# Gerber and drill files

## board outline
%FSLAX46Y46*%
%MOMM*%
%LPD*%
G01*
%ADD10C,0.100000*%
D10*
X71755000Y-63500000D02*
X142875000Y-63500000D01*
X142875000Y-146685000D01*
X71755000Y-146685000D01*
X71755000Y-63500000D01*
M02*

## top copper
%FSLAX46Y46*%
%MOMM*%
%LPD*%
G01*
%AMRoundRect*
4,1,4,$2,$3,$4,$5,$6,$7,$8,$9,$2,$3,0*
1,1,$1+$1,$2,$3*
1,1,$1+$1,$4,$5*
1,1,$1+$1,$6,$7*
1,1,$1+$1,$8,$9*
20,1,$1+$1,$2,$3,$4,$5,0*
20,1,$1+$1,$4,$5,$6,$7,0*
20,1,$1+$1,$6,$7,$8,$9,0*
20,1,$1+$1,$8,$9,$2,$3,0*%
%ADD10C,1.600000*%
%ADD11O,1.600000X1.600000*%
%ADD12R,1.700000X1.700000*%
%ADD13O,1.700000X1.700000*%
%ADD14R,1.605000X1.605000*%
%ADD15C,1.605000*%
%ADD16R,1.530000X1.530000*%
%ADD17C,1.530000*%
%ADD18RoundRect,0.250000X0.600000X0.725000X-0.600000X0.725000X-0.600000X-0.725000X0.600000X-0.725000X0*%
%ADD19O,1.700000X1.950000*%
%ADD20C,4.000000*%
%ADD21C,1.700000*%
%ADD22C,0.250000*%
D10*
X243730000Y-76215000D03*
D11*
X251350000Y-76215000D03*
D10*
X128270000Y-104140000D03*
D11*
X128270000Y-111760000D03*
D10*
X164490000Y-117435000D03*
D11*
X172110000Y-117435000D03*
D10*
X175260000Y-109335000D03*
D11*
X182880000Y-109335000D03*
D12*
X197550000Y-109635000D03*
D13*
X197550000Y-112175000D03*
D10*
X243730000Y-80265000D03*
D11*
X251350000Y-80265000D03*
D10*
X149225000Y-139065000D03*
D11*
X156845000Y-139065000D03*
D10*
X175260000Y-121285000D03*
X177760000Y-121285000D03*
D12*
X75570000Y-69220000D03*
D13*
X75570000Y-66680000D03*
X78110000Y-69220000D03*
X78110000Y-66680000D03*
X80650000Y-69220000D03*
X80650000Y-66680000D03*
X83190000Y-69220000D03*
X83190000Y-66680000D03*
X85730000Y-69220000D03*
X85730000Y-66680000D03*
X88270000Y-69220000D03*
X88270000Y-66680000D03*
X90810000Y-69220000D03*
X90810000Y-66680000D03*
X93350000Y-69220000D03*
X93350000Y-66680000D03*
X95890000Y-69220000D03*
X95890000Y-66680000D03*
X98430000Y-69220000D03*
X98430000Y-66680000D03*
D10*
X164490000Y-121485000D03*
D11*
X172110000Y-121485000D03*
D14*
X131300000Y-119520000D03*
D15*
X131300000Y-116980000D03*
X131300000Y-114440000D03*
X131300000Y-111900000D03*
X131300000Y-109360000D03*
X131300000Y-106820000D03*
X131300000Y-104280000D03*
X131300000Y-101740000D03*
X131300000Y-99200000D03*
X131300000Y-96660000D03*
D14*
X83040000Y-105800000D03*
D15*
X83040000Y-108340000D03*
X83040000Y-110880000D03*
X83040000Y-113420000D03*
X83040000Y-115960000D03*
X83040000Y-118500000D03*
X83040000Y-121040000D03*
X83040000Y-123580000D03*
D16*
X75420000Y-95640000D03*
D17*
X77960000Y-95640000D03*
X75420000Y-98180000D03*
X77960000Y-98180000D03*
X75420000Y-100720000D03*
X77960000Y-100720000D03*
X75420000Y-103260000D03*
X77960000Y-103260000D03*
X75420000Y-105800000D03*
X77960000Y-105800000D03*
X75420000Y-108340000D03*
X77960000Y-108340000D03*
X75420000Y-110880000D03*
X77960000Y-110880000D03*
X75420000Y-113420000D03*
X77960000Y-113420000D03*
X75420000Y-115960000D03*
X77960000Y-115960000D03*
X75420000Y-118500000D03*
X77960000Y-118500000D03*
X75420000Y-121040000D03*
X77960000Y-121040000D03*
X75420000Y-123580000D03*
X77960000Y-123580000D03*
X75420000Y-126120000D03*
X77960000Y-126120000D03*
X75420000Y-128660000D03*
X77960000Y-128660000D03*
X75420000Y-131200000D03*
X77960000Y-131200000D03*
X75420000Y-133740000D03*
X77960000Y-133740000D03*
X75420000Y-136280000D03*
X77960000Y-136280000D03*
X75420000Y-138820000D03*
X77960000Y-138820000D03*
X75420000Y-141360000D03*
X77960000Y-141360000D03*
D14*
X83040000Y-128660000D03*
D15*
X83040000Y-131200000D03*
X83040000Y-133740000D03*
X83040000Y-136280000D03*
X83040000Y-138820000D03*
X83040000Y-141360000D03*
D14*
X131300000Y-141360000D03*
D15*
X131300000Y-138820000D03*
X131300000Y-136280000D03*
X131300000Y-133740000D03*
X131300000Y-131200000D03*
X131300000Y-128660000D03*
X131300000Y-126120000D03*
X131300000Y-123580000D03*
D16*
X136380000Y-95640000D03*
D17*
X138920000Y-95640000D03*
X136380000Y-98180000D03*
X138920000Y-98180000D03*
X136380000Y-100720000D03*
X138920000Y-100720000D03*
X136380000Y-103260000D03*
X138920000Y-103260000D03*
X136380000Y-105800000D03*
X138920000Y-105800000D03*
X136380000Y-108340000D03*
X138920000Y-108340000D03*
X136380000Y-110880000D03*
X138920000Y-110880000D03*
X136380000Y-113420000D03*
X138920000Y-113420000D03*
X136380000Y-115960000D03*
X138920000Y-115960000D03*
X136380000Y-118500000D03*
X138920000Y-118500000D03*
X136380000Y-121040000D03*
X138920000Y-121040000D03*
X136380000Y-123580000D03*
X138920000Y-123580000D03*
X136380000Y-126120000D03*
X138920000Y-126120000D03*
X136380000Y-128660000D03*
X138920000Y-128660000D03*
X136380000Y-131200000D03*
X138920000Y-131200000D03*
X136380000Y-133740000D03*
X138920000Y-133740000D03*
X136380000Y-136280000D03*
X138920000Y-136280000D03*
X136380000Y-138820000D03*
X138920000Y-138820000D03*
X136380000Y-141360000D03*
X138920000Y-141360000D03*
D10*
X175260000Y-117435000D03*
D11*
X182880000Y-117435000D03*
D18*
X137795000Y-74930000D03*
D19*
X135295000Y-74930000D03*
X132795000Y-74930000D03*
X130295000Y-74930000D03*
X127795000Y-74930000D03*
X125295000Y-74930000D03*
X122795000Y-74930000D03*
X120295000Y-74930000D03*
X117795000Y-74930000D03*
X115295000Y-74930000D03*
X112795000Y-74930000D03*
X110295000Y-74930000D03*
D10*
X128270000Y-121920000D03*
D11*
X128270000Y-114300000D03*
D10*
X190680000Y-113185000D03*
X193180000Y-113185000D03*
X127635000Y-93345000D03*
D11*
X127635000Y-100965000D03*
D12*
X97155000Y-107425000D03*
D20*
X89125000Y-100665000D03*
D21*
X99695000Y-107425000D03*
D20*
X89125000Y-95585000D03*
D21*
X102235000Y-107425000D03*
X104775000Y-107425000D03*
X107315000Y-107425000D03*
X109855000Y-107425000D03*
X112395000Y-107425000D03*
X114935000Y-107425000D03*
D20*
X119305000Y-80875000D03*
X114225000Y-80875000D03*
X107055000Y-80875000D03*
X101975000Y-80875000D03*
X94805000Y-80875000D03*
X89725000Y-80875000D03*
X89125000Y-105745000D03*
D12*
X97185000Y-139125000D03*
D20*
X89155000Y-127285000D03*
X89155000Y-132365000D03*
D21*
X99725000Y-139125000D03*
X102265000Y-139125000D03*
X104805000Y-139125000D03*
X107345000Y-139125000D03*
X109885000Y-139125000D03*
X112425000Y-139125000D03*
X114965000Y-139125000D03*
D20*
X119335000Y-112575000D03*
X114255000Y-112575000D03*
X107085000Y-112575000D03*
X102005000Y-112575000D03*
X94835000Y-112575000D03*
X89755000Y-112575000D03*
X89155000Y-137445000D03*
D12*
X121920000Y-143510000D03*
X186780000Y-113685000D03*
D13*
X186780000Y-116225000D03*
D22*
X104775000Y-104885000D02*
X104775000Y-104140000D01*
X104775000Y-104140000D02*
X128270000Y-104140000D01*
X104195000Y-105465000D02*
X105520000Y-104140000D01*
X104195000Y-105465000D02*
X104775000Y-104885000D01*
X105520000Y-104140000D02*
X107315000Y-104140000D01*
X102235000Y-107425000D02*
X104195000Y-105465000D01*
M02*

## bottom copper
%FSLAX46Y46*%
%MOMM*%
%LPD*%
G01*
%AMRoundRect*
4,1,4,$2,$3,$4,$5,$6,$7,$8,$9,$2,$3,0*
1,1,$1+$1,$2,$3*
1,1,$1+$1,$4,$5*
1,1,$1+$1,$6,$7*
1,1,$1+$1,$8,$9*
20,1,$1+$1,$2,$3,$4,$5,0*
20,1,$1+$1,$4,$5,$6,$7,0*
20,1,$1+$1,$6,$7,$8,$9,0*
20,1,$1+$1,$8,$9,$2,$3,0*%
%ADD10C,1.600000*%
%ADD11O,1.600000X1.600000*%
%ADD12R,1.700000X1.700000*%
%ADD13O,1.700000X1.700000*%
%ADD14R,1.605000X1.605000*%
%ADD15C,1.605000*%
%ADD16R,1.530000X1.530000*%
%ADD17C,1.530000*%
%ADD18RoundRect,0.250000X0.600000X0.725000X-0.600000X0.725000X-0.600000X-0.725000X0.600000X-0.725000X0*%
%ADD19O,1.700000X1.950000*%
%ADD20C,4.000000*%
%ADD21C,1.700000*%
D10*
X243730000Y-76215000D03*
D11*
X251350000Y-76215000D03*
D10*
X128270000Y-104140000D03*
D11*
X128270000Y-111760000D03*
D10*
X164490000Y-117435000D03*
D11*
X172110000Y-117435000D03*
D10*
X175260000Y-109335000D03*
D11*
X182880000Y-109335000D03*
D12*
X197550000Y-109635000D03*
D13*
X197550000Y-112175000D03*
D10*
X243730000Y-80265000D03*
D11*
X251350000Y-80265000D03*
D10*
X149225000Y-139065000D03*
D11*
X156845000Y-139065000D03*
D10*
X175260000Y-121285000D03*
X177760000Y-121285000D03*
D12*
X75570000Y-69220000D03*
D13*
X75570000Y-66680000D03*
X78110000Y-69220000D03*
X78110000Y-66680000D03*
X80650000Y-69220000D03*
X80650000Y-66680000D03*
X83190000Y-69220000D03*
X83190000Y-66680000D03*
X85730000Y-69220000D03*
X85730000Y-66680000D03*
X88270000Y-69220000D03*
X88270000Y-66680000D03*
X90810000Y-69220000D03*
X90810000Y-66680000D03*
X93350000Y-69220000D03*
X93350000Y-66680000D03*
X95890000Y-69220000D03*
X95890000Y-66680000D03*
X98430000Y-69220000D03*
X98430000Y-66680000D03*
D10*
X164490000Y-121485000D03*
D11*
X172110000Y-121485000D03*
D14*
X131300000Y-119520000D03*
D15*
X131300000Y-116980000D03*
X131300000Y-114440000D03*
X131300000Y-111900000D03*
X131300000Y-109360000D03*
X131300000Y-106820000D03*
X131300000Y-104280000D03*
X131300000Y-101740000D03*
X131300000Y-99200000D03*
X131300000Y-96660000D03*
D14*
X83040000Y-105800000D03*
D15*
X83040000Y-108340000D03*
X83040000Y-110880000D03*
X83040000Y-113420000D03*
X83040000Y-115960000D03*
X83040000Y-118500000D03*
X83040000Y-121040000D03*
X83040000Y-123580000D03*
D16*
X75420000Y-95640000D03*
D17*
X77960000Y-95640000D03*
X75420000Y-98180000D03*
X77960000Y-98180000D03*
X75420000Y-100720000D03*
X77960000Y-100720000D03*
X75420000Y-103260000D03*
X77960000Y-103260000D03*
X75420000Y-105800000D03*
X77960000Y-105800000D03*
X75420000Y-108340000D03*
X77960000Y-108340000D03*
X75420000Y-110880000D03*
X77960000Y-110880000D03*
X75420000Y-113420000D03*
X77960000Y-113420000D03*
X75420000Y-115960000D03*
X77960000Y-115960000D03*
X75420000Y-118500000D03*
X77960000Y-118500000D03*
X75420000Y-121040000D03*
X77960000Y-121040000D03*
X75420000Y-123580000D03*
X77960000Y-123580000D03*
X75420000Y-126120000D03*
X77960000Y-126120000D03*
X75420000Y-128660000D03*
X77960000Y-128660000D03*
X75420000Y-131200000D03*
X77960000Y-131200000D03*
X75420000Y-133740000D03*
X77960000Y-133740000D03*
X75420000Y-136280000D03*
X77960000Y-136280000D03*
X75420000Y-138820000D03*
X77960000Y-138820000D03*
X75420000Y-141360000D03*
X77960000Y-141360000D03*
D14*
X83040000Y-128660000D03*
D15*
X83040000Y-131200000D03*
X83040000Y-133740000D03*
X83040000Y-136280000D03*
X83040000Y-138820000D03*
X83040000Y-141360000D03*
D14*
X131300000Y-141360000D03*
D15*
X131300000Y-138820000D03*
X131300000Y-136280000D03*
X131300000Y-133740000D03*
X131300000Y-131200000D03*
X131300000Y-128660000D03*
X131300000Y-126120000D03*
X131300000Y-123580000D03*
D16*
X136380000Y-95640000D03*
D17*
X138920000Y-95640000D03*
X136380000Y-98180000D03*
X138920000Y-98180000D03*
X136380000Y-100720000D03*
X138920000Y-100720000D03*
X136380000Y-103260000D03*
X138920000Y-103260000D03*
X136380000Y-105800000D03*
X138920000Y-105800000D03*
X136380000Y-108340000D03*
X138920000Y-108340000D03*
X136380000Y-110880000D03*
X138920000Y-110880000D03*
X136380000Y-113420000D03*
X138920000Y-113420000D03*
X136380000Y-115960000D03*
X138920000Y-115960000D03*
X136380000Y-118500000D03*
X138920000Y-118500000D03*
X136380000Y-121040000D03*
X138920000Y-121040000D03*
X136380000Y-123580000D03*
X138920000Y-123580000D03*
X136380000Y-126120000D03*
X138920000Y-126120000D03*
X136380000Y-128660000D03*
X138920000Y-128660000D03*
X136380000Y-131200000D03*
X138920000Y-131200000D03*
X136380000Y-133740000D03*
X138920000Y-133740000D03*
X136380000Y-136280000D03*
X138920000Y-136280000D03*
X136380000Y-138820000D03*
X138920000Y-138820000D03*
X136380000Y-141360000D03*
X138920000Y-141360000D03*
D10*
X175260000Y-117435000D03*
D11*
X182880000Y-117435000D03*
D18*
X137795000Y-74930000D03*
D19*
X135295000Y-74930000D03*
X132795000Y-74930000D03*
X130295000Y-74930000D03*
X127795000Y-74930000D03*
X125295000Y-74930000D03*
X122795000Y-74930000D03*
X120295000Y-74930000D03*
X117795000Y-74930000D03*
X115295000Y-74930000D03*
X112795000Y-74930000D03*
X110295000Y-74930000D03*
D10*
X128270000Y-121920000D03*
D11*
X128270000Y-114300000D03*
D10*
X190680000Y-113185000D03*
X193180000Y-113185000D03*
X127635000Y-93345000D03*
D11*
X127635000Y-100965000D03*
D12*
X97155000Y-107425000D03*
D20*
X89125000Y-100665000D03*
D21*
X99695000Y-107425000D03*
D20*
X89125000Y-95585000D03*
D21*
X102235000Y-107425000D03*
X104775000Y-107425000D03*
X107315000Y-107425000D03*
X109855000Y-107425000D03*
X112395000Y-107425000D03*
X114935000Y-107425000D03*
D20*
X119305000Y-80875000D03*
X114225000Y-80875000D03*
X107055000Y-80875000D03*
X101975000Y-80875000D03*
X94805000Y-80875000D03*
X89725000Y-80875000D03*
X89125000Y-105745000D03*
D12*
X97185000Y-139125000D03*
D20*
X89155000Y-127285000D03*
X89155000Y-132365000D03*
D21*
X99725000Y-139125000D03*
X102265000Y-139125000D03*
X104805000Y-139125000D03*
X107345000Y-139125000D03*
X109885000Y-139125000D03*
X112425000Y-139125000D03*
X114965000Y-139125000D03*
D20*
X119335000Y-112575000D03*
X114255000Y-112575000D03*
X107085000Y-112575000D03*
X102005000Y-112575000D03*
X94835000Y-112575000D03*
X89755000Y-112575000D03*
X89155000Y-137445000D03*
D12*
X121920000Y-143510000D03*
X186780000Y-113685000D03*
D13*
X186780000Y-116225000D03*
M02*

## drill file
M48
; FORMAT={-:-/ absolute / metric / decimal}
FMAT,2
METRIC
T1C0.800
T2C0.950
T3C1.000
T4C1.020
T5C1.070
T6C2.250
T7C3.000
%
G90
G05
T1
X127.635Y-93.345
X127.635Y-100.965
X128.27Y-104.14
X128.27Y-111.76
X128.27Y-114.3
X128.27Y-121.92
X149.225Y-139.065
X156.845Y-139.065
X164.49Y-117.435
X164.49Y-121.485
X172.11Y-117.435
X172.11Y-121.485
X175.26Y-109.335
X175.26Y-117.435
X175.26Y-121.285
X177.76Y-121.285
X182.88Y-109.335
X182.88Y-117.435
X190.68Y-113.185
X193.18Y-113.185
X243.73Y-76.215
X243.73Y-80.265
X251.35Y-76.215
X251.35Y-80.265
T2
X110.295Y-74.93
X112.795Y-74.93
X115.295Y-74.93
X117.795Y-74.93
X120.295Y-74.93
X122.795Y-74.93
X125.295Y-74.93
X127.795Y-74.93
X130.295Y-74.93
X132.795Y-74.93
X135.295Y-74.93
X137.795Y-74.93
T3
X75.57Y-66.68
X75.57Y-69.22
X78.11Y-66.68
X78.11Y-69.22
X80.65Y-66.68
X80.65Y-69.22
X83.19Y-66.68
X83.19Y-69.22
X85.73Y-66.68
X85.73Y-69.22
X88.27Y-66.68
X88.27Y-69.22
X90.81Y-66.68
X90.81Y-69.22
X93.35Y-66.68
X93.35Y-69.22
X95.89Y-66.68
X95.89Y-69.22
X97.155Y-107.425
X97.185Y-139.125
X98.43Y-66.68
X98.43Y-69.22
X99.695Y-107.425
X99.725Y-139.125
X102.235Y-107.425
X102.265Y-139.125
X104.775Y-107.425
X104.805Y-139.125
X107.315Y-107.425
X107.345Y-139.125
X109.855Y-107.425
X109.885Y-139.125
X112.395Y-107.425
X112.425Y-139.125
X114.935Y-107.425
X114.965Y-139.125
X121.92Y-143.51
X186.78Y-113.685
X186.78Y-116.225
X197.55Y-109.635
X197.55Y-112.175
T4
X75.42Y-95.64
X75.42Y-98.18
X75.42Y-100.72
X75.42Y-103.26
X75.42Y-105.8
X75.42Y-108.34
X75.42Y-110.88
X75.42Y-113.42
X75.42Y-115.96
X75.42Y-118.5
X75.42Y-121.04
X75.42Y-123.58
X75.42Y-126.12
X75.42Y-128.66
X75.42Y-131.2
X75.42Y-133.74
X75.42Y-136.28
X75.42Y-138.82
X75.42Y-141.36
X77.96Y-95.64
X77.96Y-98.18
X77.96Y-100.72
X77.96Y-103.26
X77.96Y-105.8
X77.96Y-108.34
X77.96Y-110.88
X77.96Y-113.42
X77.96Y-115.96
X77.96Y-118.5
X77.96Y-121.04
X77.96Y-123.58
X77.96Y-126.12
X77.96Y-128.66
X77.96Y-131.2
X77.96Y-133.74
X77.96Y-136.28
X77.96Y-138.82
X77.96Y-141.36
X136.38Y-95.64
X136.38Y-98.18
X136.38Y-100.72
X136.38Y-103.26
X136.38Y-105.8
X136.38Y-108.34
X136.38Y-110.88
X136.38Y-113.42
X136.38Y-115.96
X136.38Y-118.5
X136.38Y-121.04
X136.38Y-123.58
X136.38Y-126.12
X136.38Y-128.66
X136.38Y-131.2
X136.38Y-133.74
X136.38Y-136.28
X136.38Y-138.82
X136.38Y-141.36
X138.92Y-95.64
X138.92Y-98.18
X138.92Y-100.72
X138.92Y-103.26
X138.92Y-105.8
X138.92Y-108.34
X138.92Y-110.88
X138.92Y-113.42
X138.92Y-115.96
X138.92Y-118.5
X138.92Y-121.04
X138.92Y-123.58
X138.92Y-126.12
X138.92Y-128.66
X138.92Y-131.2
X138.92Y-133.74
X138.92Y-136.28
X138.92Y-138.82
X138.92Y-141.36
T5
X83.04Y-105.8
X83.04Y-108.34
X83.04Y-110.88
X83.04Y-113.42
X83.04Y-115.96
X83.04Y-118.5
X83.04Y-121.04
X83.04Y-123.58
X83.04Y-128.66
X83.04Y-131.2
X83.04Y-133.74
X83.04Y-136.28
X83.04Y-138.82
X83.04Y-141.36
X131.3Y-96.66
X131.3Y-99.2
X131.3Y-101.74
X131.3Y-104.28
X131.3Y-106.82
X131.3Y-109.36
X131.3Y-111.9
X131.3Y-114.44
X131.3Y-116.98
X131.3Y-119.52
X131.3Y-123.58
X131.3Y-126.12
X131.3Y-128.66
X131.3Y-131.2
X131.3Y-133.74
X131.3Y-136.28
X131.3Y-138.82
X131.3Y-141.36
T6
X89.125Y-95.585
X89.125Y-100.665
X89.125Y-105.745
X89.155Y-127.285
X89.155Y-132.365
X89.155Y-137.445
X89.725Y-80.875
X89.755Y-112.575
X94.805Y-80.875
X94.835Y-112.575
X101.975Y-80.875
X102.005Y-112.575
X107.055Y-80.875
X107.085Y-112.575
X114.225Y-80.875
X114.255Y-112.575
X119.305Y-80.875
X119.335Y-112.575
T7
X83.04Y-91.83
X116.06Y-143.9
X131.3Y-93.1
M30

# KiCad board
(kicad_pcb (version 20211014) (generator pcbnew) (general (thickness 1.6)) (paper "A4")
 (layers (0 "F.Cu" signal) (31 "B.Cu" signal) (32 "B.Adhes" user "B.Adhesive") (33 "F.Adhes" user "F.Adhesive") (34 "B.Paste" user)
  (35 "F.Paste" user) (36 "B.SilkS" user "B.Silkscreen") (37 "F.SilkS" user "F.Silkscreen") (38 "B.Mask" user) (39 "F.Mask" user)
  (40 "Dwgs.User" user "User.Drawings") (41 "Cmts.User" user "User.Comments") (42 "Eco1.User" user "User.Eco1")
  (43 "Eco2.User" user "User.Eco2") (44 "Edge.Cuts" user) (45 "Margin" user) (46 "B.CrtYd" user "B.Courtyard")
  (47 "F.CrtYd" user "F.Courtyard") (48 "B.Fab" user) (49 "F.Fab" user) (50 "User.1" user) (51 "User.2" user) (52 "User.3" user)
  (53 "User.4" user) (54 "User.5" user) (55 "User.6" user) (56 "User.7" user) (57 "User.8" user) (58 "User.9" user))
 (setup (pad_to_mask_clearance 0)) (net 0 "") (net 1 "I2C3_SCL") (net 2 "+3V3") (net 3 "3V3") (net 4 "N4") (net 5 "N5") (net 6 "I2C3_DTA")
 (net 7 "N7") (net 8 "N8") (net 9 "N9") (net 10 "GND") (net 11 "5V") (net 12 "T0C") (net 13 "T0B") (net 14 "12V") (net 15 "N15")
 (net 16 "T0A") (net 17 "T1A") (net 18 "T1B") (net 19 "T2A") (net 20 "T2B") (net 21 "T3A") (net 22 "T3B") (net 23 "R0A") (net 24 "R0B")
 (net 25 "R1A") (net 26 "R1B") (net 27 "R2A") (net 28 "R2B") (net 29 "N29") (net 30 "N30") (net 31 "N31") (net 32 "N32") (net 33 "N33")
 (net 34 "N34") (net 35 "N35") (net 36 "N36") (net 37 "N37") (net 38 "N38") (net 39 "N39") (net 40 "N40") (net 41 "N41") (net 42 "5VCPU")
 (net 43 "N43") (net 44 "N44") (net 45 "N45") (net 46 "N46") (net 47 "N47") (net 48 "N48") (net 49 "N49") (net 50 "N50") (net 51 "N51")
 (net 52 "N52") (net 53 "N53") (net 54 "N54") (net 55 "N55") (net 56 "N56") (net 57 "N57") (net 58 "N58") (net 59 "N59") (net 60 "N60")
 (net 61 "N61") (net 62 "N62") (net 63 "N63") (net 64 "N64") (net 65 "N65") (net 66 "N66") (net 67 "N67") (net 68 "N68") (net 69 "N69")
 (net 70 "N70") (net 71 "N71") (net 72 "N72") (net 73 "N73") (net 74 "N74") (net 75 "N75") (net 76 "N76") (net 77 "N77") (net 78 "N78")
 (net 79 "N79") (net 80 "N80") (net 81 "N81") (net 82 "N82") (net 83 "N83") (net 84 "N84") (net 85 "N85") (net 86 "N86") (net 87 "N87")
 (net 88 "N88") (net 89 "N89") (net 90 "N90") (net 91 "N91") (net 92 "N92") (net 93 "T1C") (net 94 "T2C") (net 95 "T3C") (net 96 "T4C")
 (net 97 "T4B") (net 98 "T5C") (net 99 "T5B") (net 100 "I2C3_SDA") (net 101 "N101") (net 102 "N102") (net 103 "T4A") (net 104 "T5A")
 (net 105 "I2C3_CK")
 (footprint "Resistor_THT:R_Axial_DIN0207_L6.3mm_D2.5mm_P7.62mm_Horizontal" (layer "F.Cu") (at 243.73 76.215)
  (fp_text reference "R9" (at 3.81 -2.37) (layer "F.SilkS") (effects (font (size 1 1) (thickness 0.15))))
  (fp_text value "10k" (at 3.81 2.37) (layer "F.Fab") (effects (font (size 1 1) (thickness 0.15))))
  (pad "1" thru_hole circle (at 0 0) (size 1.6 1.6) (drill 0.8) (layers *.Cu *.Mask) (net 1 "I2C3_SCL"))
  (pad "2" thru_hole oval (at 7.62 0) (size 1.6 1.6) (drill 0.8) (layers *.Cu *.Mask) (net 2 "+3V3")))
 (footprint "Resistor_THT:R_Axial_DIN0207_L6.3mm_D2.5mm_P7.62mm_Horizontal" (layer "F.Cu") (at 128.27 104.14 -90)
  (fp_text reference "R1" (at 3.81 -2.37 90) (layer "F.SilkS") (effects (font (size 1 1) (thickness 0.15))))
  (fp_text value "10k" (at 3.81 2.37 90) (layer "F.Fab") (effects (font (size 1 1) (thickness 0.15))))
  (pad "1" thru_hole circle (at 0 0 270) (size 1.6 1.6) (drill 0.8) (layers *.Cu *.Mask) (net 1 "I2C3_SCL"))
  (pad "2" thru_hole oval (at 7.62 0 270) (size 1.6 1.6) (drill 0.8) (layers *.Cu *.Mask) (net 2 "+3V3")))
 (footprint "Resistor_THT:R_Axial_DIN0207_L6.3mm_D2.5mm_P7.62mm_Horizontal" (layer "F.Cu") (at 164.49 117.435)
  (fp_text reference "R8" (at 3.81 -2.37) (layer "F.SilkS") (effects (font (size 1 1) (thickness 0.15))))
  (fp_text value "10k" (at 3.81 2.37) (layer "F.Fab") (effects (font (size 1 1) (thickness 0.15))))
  (pad "1" thru_hole circle (at 0 0) (size 1.6 1.6) (drill 0.8) (layers *.Cu *.Mask) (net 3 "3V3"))
  (pad "2" thru_hole oval (at 7.62 0) (size 1.6 1.6) (drill 0.8) (layers *.Cu *.Mask) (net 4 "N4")))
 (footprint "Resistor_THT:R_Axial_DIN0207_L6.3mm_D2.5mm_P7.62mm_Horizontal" (layer "F.Cu") (at 175.26 109.335)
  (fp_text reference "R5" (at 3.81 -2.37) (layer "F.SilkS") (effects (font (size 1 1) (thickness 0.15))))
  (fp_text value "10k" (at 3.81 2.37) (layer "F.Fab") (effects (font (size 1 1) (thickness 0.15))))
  (pad "1" thru_hole circle (at 0 0) (size 1.6 1.6) (drill 0.8) (layers *.Cu *.Mask) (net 3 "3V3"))
  (pad "2" thru_hole oval (at 7.62 0) (size 1.6 1.6) (drill 0.8) (layers *.Cu *.Mask) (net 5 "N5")))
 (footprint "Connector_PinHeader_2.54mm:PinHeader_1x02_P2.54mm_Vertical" (layer "F.Cu") (at 197.55 109.635)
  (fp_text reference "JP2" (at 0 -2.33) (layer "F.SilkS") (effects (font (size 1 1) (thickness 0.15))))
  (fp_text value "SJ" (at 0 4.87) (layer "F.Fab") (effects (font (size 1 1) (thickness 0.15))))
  (pad "1" thru_hole rect (at 0 0) (size 1.7 1.7) (drill 1) (layers *.Cu *.Mask) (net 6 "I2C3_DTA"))
  (pad "2" thru_hole oval (at 0 2.54) (size 1.7 1.7) (drill 1) (layers *.Cu *.Mask) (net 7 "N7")))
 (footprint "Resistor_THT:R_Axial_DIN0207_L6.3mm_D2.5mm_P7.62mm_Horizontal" (layer "F.Cu") (at 243.73 80.265)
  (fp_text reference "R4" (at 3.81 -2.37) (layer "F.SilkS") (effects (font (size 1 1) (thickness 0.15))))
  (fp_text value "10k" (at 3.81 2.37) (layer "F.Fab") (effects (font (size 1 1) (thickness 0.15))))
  (pad "1" thru_hole circle (at 0 0) (size 1.6 1.6) (drill 0.8) (layers *.Cu *.Mask) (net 3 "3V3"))
  (pad "2" thru_hole oval (at 7.62 0) (size 1.6 1.6) (drill 0.8) (layers *.Cu *.Mask) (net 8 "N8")))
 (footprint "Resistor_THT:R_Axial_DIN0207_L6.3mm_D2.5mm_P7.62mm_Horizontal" (layer "F.Cu") (at 149.225 139.065)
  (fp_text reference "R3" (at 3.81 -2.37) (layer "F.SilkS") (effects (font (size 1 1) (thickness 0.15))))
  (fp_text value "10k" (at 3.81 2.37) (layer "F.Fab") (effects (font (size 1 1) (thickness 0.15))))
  (pad "1" thru_hole circle (at 0 0) (size 1.6 1.6) (drill 0.8) (layers *.Cu *.Mask) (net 3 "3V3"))
  (pad "2" thru_hole oval (at 7.62 0) (size 1.6 1.6) (drill 0.8) (layers *.Cu *.Mask) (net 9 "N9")))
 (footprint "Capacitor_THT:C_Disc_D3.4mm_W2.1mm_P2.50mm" (layer "F.Cu") (at 175.26 121.285)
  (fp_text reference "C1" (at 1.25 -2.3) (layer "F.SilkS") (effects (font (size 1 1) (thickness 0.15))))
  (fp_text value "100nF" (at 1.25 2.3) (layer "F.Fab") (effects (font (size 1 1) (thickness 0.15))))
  (pad "1" thru_hole circle (at 0 0) (size 1.6 1.6) (drill 0.8) (layers *.Cu *.Mask) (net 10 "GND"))
  (pad "2" thru_hole circle (at 2.5 0) (size 1.6 1.6) (drill 0.8) (layers *.Cu *.Mask) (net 3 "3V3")))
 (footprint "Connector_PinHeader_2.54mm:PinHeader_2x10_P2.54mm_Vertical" (layer "F.Cu") (at 75.57 69.22 90)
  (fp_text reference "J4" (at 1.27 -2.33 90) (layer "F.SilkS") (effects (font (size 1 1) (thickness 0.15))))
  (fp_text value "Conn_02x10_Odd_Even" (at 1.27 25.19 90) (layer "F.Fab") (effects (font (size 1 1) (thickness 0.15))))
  (pad "1" thru_hole rect (at 0 0 90) (size 1.7 1.7) (drill 1) (layers *.Cu *.Mask) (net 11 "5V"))
  (pad "2" thru_hole oval (at 2.54 0 90) (size 1.7 1.7) (drill 1) (layers *.Cu *.Mask) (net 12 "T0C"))
  (pad "3" thru_hole oval (at 0 2.54 90) (size 1.7 1.7) (drill 1) (layers *.Cu *.Mask) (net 10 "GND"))
  (pad "4" thru_hole oval (at 2.54 2.54 90) (size 1.7 1.7) (drill 1) (layers *.Cu *.Mask) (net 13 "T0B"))
  (pad "5" thru_hole oval (at 0 5.08 90) (size 1.7 1.7) (drill 1) (layers *.Cu *.Mask) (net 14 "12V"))
  (pad "6" thru_hole oval (at 2.54 5.08 90) (size 1.7 1.7) (drill 1) (layers *.Cu *.Mask) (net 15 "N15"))
  (pad "7" thru_hole oval (at 0 7.62 90) (size 1.7 1.7) (drill 1) (layers *.Cu *.Mask) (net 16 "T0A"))
  (pad "8" thru_hole oval (at 2.54 7.62 90) (size 1.7 1.7) (drill 1) (layers *.Cu *.Mask) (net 13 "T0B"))
  (pad "9" thru_hole oval (at 0 10.16 90) (size 1.7 1.7) (drill 1) (layers *.Cu *.Mask) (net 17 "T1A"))
  (pad "10" thru_hole oval (at 2.54 10.16 90) (size 1.7 1.7) (drill 1) (layers *.Cu *.Mask) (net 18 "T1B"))
  (pad "11" thru_hole oval (at 0 12.7 90) (size 1.7 1.7) (drill 1) (layers *.Cu *.Mask) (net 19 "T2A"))
  (pad "12" thru_hole oval (at 2.54 12.7 90) (size 1.7 1.7) (drill 1) (layers *.Cu *.Mask) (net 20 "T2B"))
  (pad "13" thru_hole oval (at 0 15.24 90) (size 1.7 1.7) (drill 1) (layers *.Cu *.Mask) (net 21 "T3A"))
  (pad "14" thru_hole oval (at 2.54 15.24 90) (size 1.7 1.7) (drill 1) (layers *.Cu *.Mask) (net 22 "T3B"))
  (pad "15" thru_hole oval (at 0 17.78 90) (size 1.7 1.7) (drill 1) (layers *.Cu *.Mask) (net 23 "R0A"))
  (pad "16" thru_hole oval (at 2.54 17.78 90) (size 1.7 1.7) (drill 1) (layers *.Cu *.Mask) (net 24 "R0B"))
  (pad "17" thru_hole oval (at 0 20.32 90) (size 1.7 1.7) (drill 1) (layers *.Cu *.Mask) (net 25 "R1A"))
  (pad "18" thru_hole oval (at 2.54 20.32 90) (size 1.7 1.7) (drill 1) (layers *.Cu *.Mask) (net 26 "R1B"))
  (pad "19" thru_hole oval (at 0 22.86 90) (size 1.7 1.7) (drill 1) (layers *.Cu *.Mask) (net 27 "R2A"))
  (pad "20" thru_hole oval (at 2.54 22.86 90) (size 1.7 1.7) (drill 1) (layers *.Cu *.Mask) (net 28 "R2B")))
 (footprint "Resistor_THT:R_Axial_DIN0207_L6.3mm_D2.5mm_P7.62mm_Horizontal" (layer "F.Cu") (at 164.49 121.485)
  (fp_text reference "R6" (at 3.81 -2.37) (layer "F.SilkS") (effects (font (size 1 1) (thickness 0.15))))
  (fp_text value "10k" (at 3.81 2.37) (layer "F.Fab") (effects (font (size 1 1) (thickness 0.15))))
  (pad "1" thru_hole circle (at 0 0) (size 1.6 1.6) (drill 0.8) (layers *.Cu *.Mask) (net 3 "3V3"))
  (pad "2" thru_hole oval (at 7.62 0) (size 1.6 1.6) (drill 0.8) (layers *.Cu *.Mask) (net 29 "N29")))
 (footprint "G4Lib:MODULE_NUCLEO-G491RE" (layer "F.Cu") (at 107.17 105.15)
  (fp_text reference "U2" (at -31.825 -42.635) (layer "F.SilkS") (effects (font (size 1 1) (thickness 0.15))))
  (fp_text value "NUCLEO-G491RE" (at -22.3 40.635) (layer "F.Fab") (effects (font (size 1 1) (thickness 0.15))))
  (pad "" np_thru_hole circle (at -24.13 -13.32) (size 3 3) (drill 3) (layers *.Cu *.Mask))
  (pad "" np_thru_hole circle (at 24.13 -12.05) (size 3 3) (drill 3) (layers *.Cu *.Mask))
  (pad "" np_thru_hole circle (at 8.89 38.75) (size 3 3) (drill 3) (layers *.Cu *.Mask))
  (pad "CN5_1" thru_hole rect (at 24.13 14.37) (size 1.605 1.605) (drill 1.07) (layers *.Cu *.Mask))
  (pad "CN5_2" thru_hole circle (at 24.13 11.83) (size 1.605 1.605) (drill 1.07) (layers *.Cu *.Mask))
  (pad "CN5_3" thru_hole circle (at 24.13 9.29) (size 1.605 1.605) (drill 1.07) (layers *.Cu *.Mask))
  (pad "CN5_4" thru_hole circle (at 24.13 6.75) (size 1.605 1.605) (drill 1.07) (layers *.Cu *.Mask))
  (pad "CN5_5" thru_hole circle (at 24.13 4.21) (size 1.605 1.605) (drill 1.07) (layers *.Cu *.Mask))
  (pad "CN5_6" thru_hole circle (at 24.13 1.67) (size 1.605 1.605) (drill 1.07) (layers *.Cu *.Mask))
  (pad "CN5_7" thru_hole circle (at 24.13 -0.87) (size 1.605 1.605) (drill 1.07) (layers *.Cu *.Mask))
  (pad "CN5_8" thru_hole circle (at 24.13 -3.41) (size 1.605 1.605) (drill 1.07) (layers *.Cu *.Mask))
  (pad "CN5_9" thru_hole circle (at 24.13 -5.95) (size 1.605 1.605) (drill 1.07) (layers *.Cu *.Mask))
  (pad "CN5_10" thru_hole circle (at 24.13 -8.49) (size 1.605 1.605) (drill 1.07) (layers *.Cu *.Mask))
  (pad "CN6_1" thru_hole rect (at -24.13 0.65) (size 1.605 1.605) (drill 1.07) (layers *.Cu *.Mask))
  (pad "CN6_2" thru_hole circle (at -24.13 3.19) (size 1.605 1.605) (drill 1.07) (layers *.Cu *.Mask))
  (pad "CN6_3" thru_hole circle (at -24.13 5.73) (size 1.605 1.605) (drill 1.07) (layers *.Cu *.Mask))
  (pad "CN6_4" thru_hole circle (at -24.13 8.27) (size 1.605 1.605) (drill 1.07) (layers *.Cu *.Mask))
  (pad "CN6_5" thru_hole circle (at -24.13 10.81) (size 1.605 1.605) (drill 1.07) (layers *.Cu *.Mask))
  (pad "CN6_6" thru_hole circle (at -24.13 13.35) (size 1.605 1.605) (drill 1.07) (layers *.Cu *.Mask))
  (pad "CN6_7" thru_hole circle (at -24.13 15.89) (size 1.605 1.605) (drill 1.07) (layers *.Cu *.Mask))
  (pad "CN6_8" thru_hole circle (at -24.13 18.43) (size 1.605 1.605) (drill 1.07) (layers *.Cu *.Mask))
  (pad "CN7_1" thru_hole rect (at -31.75 -9.51) (size 1.53 1.53) (drill 1.02) (layers *.Cu *.Mask) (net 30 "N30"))
  (pad "CN7_2" thru_hole circle (at -29.21 -9.51) (size 1.53 1.53) (drill 1.02) (layers *.Cu *.Mask) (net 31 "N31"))
  (pad "CN7_3" thru_hole circle (at -31.75 -6.97) (size 1.53 1.53) (drill 1.02) (layers *.Cu *.Mask) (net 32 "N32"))
  (pad "CN7_4" thru_hole circle (at -29.21 -6.97) (size 1.53 1.53) (drill 1.02) (layers *.Cu *.Mask) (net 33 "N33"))
  (pad "CN7_5" thru_hole circle (at -31.75 -4.43) (size 1.53 1.53) (drill 1.02) (layers *.Cu *.Mask) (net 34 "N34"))
  (pad "CN7_6" thru_hole circle (at -29.21 -4.43) (size 1.53 1.53) (drill 1.02) (layers *.Cu *.Mask) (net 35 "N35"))
  (pad "CN7_7" thru_hole circle (at -31.75 -1.89) (size 1.53 1.53) (drill 1.02) (layers *.Cu *.Mask) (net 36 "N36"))
  (pad "CN7_8" thru_hole circle (at -29.21 -1.89) (size 1.53 1.53) (drill 1.02) (layers *.Cu *.Mask) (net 10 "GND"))
  (pad "CN7_9" thru_hole circle (at -31.75 0.65) (size 1.53 1.53) (drill 1.02) (layers *.Cu *.Mask))
  (pad "CN7_10" thru_hole circle (at -29.21 0.65) (size 1.53 1.53) (drill 1.02) (layers *.Cu *.Mask))
  (pad "CN7_11" thru_hole circle (at -31.75 3.19) (size 1.53 1.53) (drill 1.02) (layers *.Cu *.Mask))
  (pad "CN7_12" thru_hole circle (at -29.21 3.19) (size 1.53 1.53) (drill 1.02) (layers *.Cu *.Mask) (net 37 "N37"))
  (pad "CN7_13" thru_hole circle (at -31.75 5.73) (size 1.53 1.53) (drill 1.02) (layers *.Cu *.Mask) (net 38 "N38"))
  (pad "CN7_14" thru_hole circle (at -29.21 5.73) (size 1.53 1.53) (drill 1.02) (layers *.Cu *.Mask) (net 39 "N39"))
  (pad "CN7_15" thru_hole circle (at -31.75 8.27) (size 1.53 1.53) (drill 1.02) (layers *.Cu *.Mask) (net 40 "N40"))
  (pad "CN7_16" thru_hole circle (at -29.21 8.27) (size 1.53 1.53) (drill 1.02) (layers *.Cu *.Mask) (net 3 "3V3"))
  (pad "CN7_17" thru_hole circle (at -31.75 10.81) (size 1.53 1.53) (drill 1.02) (layers *.Cu *.Mask) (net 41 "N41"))
  (pad "CN7_18" thru_hole circle (at -29.21 10.81) (size 1.53 1.53) (drill 1.02) (layers *.Cu *.Mask) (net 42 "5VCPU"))
  (pad "CN7_19" thru_hole circle (at -31.75 13.35) (size 1.53 1.53) (drill 1.02) (layers *.Cu *.Mask) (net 10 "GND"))
  (pad "CN7_20" thru_hole circle (at -29.21 13.35) (size 1.53 1.53) (drill 1.02) (layers *.Cu *.Mask) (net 10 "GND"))
  (pad "CN7_21" thru_hole circle (at -31.75 15.89) (size 1.53 1.53) (drill 1.02) (layers *.Cu *.Mask) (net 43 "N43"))
  (pad "CN7_22" thru_hole circle (at -29.21 15.89) (size 1.53 1.53) (drill 1.02) (layers *.Cu *.Mask) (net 10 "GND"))
  (pad "CN7_23" thru_hole circle (at -31.75 18.43) (size 1.53 1.53) (drill 1.02) (layers *.Cu *.Mask) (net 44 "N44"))
  (pad "CN7_24" thru_hole circle (at -29.21 18.43) (size 1.53 1.53) (drill 1.02) (layers *.Cu *.Mask) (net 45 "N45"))
  (pad "CN7_25" thru_hole circle (at -31.75 20.97) (size 1.53 1.53) (drill 1.02) (layers *.Cu *.Mask) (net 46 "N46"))
  (pad "CN7_26" thru_hole circle (at -29.21 20.97) (size 1.53 1.53) (drill 1.02) (layers *.Cu *.Mask))
  (pad "CN7_27" thru_hole circle (at -31.75 23.51) (size 1.53 1.53) (drill 1.02) (layers *.Cu *.Mask) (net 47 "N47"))
  (pad "CN7_28" thru_hole circle (at -29.21 23.51) (size 1.53 1.53) (drill 1.02) (layers *.Cu *.Mask) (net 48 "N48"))
  (pad "CN7_29" thru_hole circle (at -31.75 26.05) (size 1.53 1.53) (drill 1.02) (layers *.Cu *.Mask) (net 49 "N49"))
  (pad "CN7_30" thru_hole circle (at -29.21 26.05) (size 1.53 1.53) (drill 1.02) (layers *.Cu *.Mask) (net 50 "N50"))
  (pad "CN7_31" thru_hole circle (at -31.75 28.59) (size 1.53 1.53) (drill 1.02) (layers *.Cu *.Mask) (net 10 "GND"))
  (pad "CN7_32" thru_hole circle (at -29.21 28.59) (size 1.53 1.53) (drill 1.02) (layers *.Cu *.Mask) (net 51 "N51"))
  (pad "CN7_33" thru_hole circle (at -31.75 31.13) (size 1.53 1.53) (drill 1.02) (layers *.Cu *.Mask) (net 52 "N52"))
  (pad "CN7_34" thru_hole circle (at -29.21 31.13) (size 1.53 1.53) (drill 1.02) (layers *.Cu *.Mask) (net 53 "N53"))
  (pad "CN7_35" thru_hole circle (at -31.75 33.67) (size 1.53 1.53) (drill 1.02) (layers *.Cu *.Mask) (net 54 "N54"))
  (pad "CN7_36" thru_hole circle (at -29.21 33.67) (size 1.53 1.53) (drill 1.02) (layers *.Cu *.Mask) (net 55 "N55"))
  (pad "CN7_37" thru_hole circle (at -31.75 36.21) (size 1.53 1.53) (drill 1.02) (layers *.Cu *.Mask) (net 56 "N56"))
  (pad "CN7_38" thru_hole circle (at -29.21 36.21) (size 1.53 1.53) (drill 1.02) (layers *.Cu *.Mask) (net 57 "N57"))
  (pad "CN8_1" thru_hole rect (at -24.13 23.51) (size 1.605 1.605) (drill 1.07) (layers *.Cu *.Mask))
  (pad "CN8_2" thru_hole circle (at -24.13 26.05) (size 1.605 1.605) (drill 1.07) (layers *.Cu *.Mask))
  (pad "CN8_3" thru_hole circle (at -24.13 28.59) (size 1.605 1.605) (drill 1.07) (layers *.Cu *.Mask))
  (pad "CN8_4" thru_hole circle (at -24.13 31.13) (size 1.605 1.605) (drill 1.07) (layers *.Cu *.Mask))
  (pad "CN8_5" thru_hole circle (at -24.13 33.67) (size 1.605 1.605) (drill 1.07) (layers *.Cu *.Mask))
  (pad "CN8_6" thru_hole circle (at -24.13 36.21) (size 1.605 1.605) (drill 1.07) (layers *.Cu *.Mask))
  (pad "CN9_1" thru_hole rect (at 24.13 36.21) (size 1.605 1.605) (drill 1.07) (layers *.Cu *.Mask))
  (pad "CN9_2" thru_hole circle (at 24.13 33.67) (size 1.605 1.605) (drill 1.07) (layers *.Cu *.Mask))
  (pad "CN9_3" thru_hole circle (at 24.13 31.13) (size 1.605 1.605) (drill 1.07) (layers *.Cu *.Mask))
  (pad "CN9_4" thru_hole circle (at 24.13 28.59) (size 1.605 1.605) (drill 1.07) (layers *.Cu *.Mask))
  (pad "CN9_5" thru_hole circle (at 24.13 26.05) (size 1.605 1.605) (drill 1.07) (layers *.Cu *.Mask))
  (pad "CN9_6" thru_hole circle (at 24.13 23.51) (size 1.605 1.605) (drill 1.07) (layers *.Cu *.Mask))
  (pad "CN9_7" thru_hole circle (at 24.13 20.97) (size 1.605 1.605) (drill 1.07) (layers *.Cu *.Mask))
  (pad "CN9_8" thru_hole circle (at 24.13 18.43) (size 1.605 1.605) (drill 1.07) (layers *.Cu *.Mask))
  (pad "CN10_1" thru_hole rect (at 29.21 -9.51) (size 1.53 1.53) (drill 1.02) (layers *.Cu *.Mask) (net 7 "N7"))
  (pad "CN10_2" thru_hole circle (at 31.75 -9.51) (size 1.53 1.53) (drill 1.02) (layers *.Cu *.Mask) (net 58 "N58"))
  (pad "CN10_3" thru_hole circle (at 29.21 -6.97) (size 1.53 1.53) (drill 1.02) (layers *.Cu *.Mask) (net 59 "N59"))
  (pad "CN10_4" thru_hole circle (at 31.75 -6.97) (size 1.53 1.53) (drill 1.02) (layers *.Cu *.Mask) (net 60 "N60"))
  (pad "CN10_5" thru_hole circle (at 29.21 -4.43) (size 1.53 1.53) (drill 1.02) (layers *.Cu *.Mask) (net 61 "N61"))
  (pad "CN10_6" thru_hole circle (at 31.75 -4.43) (size 1.53 1.53) (drill 1.02) (layers *.Cu *.Mask) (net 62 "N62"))
  (pad "CN10_7" thru_hole circle (at 29.21 -1.89) (size 1.53 1.53) (drill 1.02) (layers *.Cu *.Mask) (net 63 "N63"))
  (pad "CN10_8" thru_hole circle (at 31.75 -1.89) (size 1.53 1.53) (drill 1.02) (layers *.Cu *.Mask) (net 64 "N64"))
  (pad "CN10_9" thru_hole circle (at 29.21 0.65) (size 1.53 1.53) (drill 1.02) (layers *.Cu *.Mask) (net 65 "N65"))
  (pad "CN10_10" thru_hole circle (at 31.75 0.65) (size 1.53 1.53) (drill 1.02) (layers *.Cu *.Mask))
  (pad "CN10_11" thru_hole circle (at 29.21 3.19) (size 1.53 1.53) (drill 1.02) (layers *.Cu *.Mask) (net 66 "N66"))
  (pad "CN10_12" thru_hole circle (at 31.75 3.19) (size 1.53 1.53) (drill 1.02) (layers *.Cu *.Mask) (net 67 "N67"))
  (pad "CN10_13" thru_hole circle (at 29.21 5.73) (size 1.53 1.53) (drill 1.02) (layers *.Cu *.Mask) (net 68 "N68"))
  (pad "CN10_14" thru_hole circle (at 31.75 5.73) (size 1.53 1.53) (drill 1.02) (layers *.Cu *.Mask) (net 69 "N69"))
  (pad "CN10_15" thru_hole circle (at 29.21 8.27) (size 1.53 1.53) (drill 1.02) (layers *.Cu *.Mask) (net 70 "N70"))
  (pad "CN10_16" thru_hole circle (at 31.75 8.27) (size 1.53 1.53) (drill 1.02) (layers *.Cu *.Mask) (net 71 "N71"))
  (pad "CN10_17" thru_hole circle (at 29.21 10.81) (size 1.53 1.53) (drill 1.02) (layers *.Cu *.Mask) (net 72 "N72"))
  (pad "CN10_18" thru_hole circle (at 31.75 10.81) (size 1.53 1.53) (drill 1.02) (layers *.Cu *.Mask) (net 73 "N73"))
  (pad "CN10_19" thru_hole circle (at 29.21 13.35) (size 1.53 1.53) (drill 1.02) (layers *.Cu *.Mask) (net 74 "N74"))
  (pad "CN10_20" thru_hole circle (at 31.75 13.35) (size 1.53 1.53) (drill 1.02) (layers *.Cu *.Mask) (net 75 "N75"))
  (pad "CN10_21" thru_hole circle (at 29.21 15.89) (size 1.53 1.53) (drill 1.02) (layers *.Cu *.Mask) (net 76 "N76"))
  (pad "CN10_22" thru_hole circle (at 31.75 15.89) (size 1.53 1.53) (drill 1.02) (layers *.Cu *.Mask) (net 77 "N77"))
  (pad "CN10_23" thru_hole circle (at 29.21 18.43) (size 1.53 1.53) (drill 1.02) (layers *.Cu *.Mask) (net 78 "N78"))
  (pad "CN10_24" thru_hole circle (at 31.75 18.43) (size 1.53 1.53) (drill 1.02) (layers *.Cu *.Mask) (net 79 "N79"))
  (pad "CN10_25" thru_hole circle (at 29.21 20.97) (size 1.53 1.53) (drill 1.02) (layers *.Cu *.Mask) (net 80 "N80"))
  (pad "CN10_26" thru_hole circle (at 31.75 20.97) (size 1.53 1.53) (drill 1.02) (layers *.Cu *.Mask) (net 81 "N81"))
  (pad "CN10_27" thru_hole circle (at 29.21 23.51) (size 1.53 1.53) (drill 1.02) (layers *.Cu *.Mask) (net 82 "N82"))
  (pad "CN10_28" thru_hole circle (at 31.75 23.51) (size 1.53 1.53) (drill 1.02) (layers *.Cu *.Mask) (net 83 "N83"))
  (pad "CN10_29" thru_hole circle (at 29.21 26.05) (size 1.53 1.53) (drill 1.02) (layers *.Cu *.Mask) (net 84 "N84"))
  (pad "CN10_30" thru_hole circle (at 31.75 26.05) (size 1.53 1.53) (drill 1.02) (layers *.Cu *.Mask) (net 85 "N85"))
  (pad "CN10_31" thru_hole circle (at 29.21 28.59) (size 1.53 1.53) (drill 1.02) (layers *.Cu *.Mask) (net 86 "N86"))
  (pad "CN10_32" thru_hole circle (at 31.75 28.59) (size 1.53 1.53) (drill 1.02) (layers *.Cu *.Mask) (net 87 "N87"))
  (pad "CN10_33" thru_hole circle (at 29.21 31.13) (size 1.53 1.53) (drill 1.02) (layers *.Cu *.Mask) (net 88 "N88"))
  (pad "CN10_34" thru_hole circle (at 31.75 31.13) (size 1.53 1.53) (drill 1.02) (layers *.Cu *.Mask) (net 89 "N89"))
  (pad "CN10_35" thru_hole circle (at 29.21 33.67) (size 1.53 1.53) (drill 1.02) (layers *.Cu *.Mask) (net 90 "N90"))
  (pad "CN10_36" thru_hole circle (at 31.75 33.67) (size 1.53 1.53) (drill 1.02) (layers *.Cu *.Mask))
  (pad "CN10_37" thru_hole circle (at 29.21 36.21) (size 1.53 1.53) (drill 1.02) (layers *.Cu *.Mask) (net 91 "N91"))
  (pad "CN10_38" thru_hole circle (at 31.75 36.21) (size 1.53 1.53) (drill 1.02) (layers *.Cu *.Mask)))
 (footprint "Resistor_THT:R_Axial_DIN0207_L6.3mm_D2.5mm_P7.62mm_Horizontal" (layer "F.Cu") (at 175.26 117.435)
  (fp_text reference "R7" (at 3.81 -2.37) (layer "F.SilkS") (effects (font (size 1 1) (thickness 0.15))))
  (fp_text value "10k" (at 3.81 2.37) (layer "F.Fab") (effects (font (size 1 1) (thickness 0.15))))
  (pad "1" thru_hole circle (at 0 0) (size 1.6 1.6) (drill 0.8) (layers *.Cu *.Mask) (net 3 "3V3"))
  (pad "2" thru_hole oval (at 7.62 0) (size 1.6 1.6) (drill 0.8) (layers *.Cu *.Mask) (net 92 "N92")))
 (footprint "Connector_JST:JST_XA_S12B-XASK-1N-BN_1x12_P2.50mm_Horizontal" (layer "F.Cu") (at 137.795 74.93 180)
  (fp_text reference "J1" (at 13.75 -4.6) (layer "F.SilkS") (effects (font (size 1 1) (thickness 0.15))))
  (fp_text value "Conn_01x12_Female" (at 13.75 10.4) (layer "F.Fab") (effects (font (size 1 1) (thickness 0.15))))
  (pad "1" thru_hole roundrect (at 0 0 180) (size 1.7 1.95) (drill 0.95) (layers *.Cu *.Mask) (roundrect_rratio 0.147059) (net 12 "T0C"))
  (pad "2" thru_hole oval (at 2.5 0 180) (size 1.7 1.95) (drill 0.95) (layers *.Cu *.Mask) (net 13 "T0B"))
  (pad "3" thru_hole oval (at 5 0 180) (size 1.7 1.95) (drill 0.95) (layers *.Cu *.Mask) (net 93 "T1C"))
  (pad "4" thru_hole oval (at 7.5 0 180) (size 1.7 1.95) (drill 0.95) (layers *.Cu *.Mask) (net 18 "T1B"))
  (pad "5" thru_hole oval (at 10 0 180) (size 1.7 1.95) (drill 0.95) (layers *.Cu *.Mask) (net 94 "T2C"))
  (pad "6" thru_hole oval (at 12.5 0 180) (size 1.7 1.95) (drill 0.95) (layers *.Cu *.Mask) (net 20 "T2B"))
  (pad "7" thru_hole oval (at 15 0 180) (size 1.7 1.95) (drill 0.95) (layers *.Cu *.Mask) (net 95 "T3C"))
  (pad "8" thru_hole oval (at 17.5 0 180) (size 1.7 1.95) (drill 0.95) (layers *.Cu *.Mask) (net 22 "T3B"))
  (pad "9" thru_hole oval (at 20 0 180) (size 1.7 1.95) (drill 0.95) (layers *.Cu *.Mask) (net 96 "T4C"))
  (pad "10" thru_hole oval (at 22.5 0 180) (size 1.7 1.95) (drill 0.95) (layers *.Cu *.Mask) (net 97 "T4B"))
  (pad "11" thru_hole oval (at 25 0 180) (size 1.7 1.95) (drill 0.95) (layers *.Cu *.Mask) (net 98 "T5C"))
  (pad "12" thru_hole oval (at 27.5 0 180) (size 1.7 1.95) (drill 0.95) (layers *.Cu *.Mask) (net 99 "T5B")))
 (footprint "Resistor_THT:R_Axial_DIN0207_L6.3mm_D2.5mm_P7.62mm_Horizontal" (layer "F.Cu") (at 128.27 121.92 90)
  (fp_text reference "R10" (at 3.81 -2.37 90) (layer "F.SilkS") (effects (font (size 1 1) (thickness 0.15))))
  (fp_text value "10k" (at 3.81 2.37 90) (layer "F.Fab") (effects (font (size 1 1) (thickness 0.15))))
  (pad "1" thru_hole circle (at 0 0 90) (size 1.6 1.6) (drill 0.8) (layers *.Cu *.Mask) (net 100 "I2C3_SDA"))
  (pad "2" thru_hole oval (at 7.62 0 90) (size 1.6 1.6) (drill 0.8) (layers *.Cu *.Mask) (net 2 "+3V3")))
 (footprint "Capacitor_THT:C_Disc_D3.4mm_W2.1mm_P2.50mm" (layer "F.Cu") (at 190.68 113.185)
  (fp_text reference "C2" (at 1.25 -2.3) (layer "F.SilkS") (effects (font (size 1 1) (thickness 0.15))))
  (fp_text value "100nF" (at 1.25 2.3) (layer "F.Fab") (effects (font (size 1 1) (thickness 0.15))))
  (pad "1" thru_hole circle (at 0 0) (size 1.6 1.6) (drill 0.8) (layers *.Cu *.Mask) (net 10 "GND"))
  (pad "2" thru_hole circle (at 2.5 0) (size 1.6 1.6) (drill 0.8) (layers *.Cu *.Mask) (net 3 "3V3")))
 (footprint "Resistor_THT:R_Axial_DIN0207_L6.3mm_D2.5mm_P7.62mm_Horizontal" (layer "F.Cu") (at 127.635 93.345 -90)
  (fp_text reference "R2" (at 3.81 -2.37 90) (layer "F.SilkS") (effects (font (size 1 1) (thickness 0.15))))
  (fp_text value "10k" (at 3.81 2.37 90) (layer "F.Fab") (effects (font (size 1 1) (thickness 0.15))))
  (pad "1" thru_hole circle (at 0 0 270) (size 1.6 1.6) (drill 0.8) (layers *.Cu *.Mask) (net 100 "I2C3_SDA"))
  (pad "2" thru_hole oval (at 7.62 0 270) (size 1.6 1.6) (drill 0.8) (layers *.Cu *.Mask) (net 2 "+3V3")))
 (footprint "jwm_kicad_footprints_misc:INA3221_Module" (layer "F.Cu") (at 97.125 107.365 180)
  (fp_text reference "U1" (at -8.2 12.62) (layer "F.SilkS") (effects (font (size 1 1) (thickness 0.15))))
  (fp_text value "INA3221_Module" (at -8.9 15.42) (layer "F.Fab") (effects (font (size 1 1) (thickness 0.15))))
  (pad "1" thru_hole rect locked (at -0.03 -0.06) (size 1.7 1.7) (drill 1) (layers *.Cu *.Mask) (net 3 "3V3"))
  (pad "2" thru_hole circle locked (at 8 6.7) (size 4 4) (drill 2.25) (layers *.Cu *.Mask) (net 10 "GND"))
  (pad "2" thru_hole circle locked (at -2.57 -0.06) (size 1.7 1.7) (drill 1) (layers *.Cu *.Mask) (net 10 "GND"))
  (pad "2" thru_hole circle locked (at 8 11.78) (size 4 4) (drill 2.25) (layers *.Cu *.Mask) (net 10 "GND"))
  (pad "3" thru_hole circle locked (at -5.11 -0.06) (size 1.7 1.7) (drill 1) (layers *.Cu *.Mask) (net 1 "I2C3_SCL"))
  (pad "4" thru_hole circle locked (at -7.65 -0.06) (size 1.7 1.7) (drill 1) (layers *.Cu *.Mask) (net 100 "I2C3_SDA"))
  (pad "5" thru_hole circle locked (at -10.19 -0.06) (size 1.7 1.7) (drill 1) (layers *.Cu *.Mask) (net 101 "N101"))
  (pad "6" thru_hole circle locked (at -12.73 -0.06) (size 1.7 1.7) (drill 1) (layers *.Cu *.Mask) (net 9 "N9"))
  (pad "7" thru_hole circle locked (at -15.27 -0.06) (size 1.7 1.7) (drill 1) (layers *.Cu *.Mask) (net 8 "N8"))
  (pad "8" thru_hole circle locked (at -17.81 -0.06) (size 1.7 1.7) (drill 1) (layers *.Cu *.Mask) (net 5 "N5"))
  (pad "9" thru_hole circle locked (at -22.18 26.49) (size 4 4) (drill 2.25) (layers *.Cu *.Mask) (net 16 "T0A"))
  (pad "10" thru_hole circle locked (at -17.1 26.49) (size 4 4) (drill 2.25) (layers *.Cu *.Mask) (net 12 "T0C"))
  (pad "11" thru_hole circle locked (at -9.93 26.49) (size 4 4) (drill 2.25) (layers *.Cu *.Mask) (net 17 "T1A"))
  (pad "12" thru_hole circle locked (at -4.85 26.49) (size 4 4) (drill 2.25) (layers *.Cu *.Mask) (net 93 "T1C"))
  (pad "13" thru_hole circle locked (at 2.32 26.49) (size 4 4) (drill 2.25) (layers *.Cu *.Mask) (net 19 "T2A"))
  (pad "14" thru_hole circle locked (at 7.4 26.49) (size 4 4) (drill 2.25) (layers *.Cu *.Mask) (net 94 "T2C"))
  (pad "15" thru_hole circle locked (at 8 1.62) (size 4 4) (drill 2.25) (layers *.Cu *.Mask) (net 3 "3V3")))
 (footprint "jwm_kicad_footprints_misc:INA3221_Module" (layer "F.Cu") (at 97.155 139.065 180)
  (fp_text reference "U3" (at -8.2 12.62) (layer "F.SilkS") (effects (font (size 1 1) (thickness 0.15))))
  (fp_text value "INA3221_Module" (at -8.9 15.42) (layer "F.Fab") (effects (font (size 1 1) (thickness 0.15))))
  (pad "1" thru_hole rect locked (at -0.03 -0.06) (size 1.7 1.7) (drill 1) (layers *.Cu *.Mask) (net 3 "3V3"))
  (pad "2" thru_hole circle locked (at 8 11.78) (size 4 4) (drill 2.25) (layers *.Cu *.Mask) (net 10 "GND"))
  (pad "2" thru_hole circle locked (at 8 6.7) (size 4 4) (drill 2.25) (layers *.Cu *.Mask) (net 10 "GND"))
  (pad "2" thru_hole circle locked (at -2.57 -0.06) (size 1.7 1.7) (drill 1) (layers *.Cu *.Mask) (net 10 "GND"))
  (pad "3" thru_hole circle locked (at -5.11 -0.06) (size 1.7 1.7) (drill 1) (layers *.Cu *.Mask) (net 1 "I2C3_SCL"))
  (pad "4" thru_hole circle locked (at -7.65 -0.06) (size 1.7 1.7) (drill 1) (layers *.Cu *.Mask) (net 100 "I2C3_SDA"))
  (pad "5" thru_hole circle locked (at -10.19 -0.06) (size 1.7 1.7) (drill 1) (layers *.Cu *.Mask) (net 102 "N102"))
  (pad "6" thru_hole circle locked (at -12.73 -0.06) (size 1.7 1.7) (drill 1) (layers *.Cu *.Mask) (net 29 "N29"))
  (pad "7" thru_hole circle locked (at -15.27 -0.06) (size 1.7 1.7) (drill 1) (layers *.Cu *.Mask) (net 92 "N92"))
  (pad "8" thru_hole circle locked (at -17.81 -0.06) (size 1.7 1.7) (drill 1) (layers *.Cu *.Mask) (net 4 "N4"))
  (pad "9" thru_hole circle locked (at -22.18 26.49) (size 4 4) (drill 2.25) (layers *.Cu *.Mask) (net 21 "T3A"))
  (pad "10" thru_hole circle locked (at -17.1 26.49) (size 4 4) (drill 2.25) (layers *.Cu *.Mask) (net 95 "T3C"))
  (pad "11" thru_hole circle locked (at -9.93 26.49) (size 4 4) (drill 2.25) (layers *.Cu *.Mask) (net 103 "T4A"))
  (pad "12" thru_hole circle locked (at -4.85 26.49) (size 4 4) (drill 2.25) (layers *.Cu *.Mask) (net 96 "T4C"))
  (pad "13" thru_hole circle locked (at 2.32 26.49) (size 4 4) (drill 2.25) (layers *.Cu *.Mask) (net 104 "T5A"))
  (pad "14" thru_hole circle locked (at 7.4 26.49) (size 4 4) (drill 2.25) (layers *.Cu *.Mask) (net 98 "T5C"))
  (pad "15" thru_hole circle locked (at 8 1.62) (size 4 4) (drill 2.25) (layers *.Cu *.Mask) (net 3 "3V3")))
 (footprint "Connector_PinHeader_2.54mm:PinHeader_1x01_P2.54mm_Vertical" (layer "F.Cu") (at 121.92 143.51)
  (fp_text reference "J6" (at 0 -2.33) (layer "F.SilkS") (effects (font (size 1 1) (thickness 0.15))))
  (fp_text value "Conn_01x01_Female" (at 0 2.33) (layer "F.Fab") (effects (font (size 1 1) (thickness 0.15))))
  (pad "1" thru_hole rect (at 0 0) (size 1.7 1.7) (drill 1) (layers *.Cu *.Mask) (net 10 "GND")))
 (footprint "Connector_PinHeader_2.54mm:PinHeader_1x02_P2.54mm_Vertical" (layer "F.Cu") (at 186.78 113.685)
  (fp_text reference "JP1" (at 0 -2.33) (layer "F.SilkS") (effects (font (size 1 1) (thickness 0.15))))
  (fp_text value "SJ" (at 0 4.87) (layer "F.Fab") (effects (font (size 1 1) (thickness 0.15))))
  (pad "1" thru_hole rect (at 0 0) (size 1.7 1.7) (drill 1) (layers *.Cu *.Mask) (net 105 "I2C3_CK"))
  (pad "2" thru_hole oval (at 0 2.54) (size 1.7 1.7) (drill 1) (layers *.Cu *.Mask) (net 58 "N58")))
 (gr_rect (start 71.755 63.5) (end 142.875 146.685) (layer "Edge.Cuts") (width 0.1) (fill none))
 (segment (start 104.775 104.885) (end 104.775 104.14) (width 0.25) (layer "F.Cu") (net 1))
 (segment (start 104.775 104.14) (end 128.27 104.14) (width 0.25) (layer "F.Cu") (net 1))
 (segment (start 104.195 105.465) (end 105.52 104.14) (width 0.25) (layer "F.Cu") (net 1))
 (segment (start 104.195 105.465) (end 104.775 104.885) (width 0.25) (layer "F.Cu") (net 1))
 (segment (start 105.52 104.14) (end 107.315 104.14) (width 0.25) (layer "F.Cu") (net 1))
 (segment (start 102.235 107.425) (end 104.195 105.465) (width 0.25) (layer "F.Cu") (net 1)))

